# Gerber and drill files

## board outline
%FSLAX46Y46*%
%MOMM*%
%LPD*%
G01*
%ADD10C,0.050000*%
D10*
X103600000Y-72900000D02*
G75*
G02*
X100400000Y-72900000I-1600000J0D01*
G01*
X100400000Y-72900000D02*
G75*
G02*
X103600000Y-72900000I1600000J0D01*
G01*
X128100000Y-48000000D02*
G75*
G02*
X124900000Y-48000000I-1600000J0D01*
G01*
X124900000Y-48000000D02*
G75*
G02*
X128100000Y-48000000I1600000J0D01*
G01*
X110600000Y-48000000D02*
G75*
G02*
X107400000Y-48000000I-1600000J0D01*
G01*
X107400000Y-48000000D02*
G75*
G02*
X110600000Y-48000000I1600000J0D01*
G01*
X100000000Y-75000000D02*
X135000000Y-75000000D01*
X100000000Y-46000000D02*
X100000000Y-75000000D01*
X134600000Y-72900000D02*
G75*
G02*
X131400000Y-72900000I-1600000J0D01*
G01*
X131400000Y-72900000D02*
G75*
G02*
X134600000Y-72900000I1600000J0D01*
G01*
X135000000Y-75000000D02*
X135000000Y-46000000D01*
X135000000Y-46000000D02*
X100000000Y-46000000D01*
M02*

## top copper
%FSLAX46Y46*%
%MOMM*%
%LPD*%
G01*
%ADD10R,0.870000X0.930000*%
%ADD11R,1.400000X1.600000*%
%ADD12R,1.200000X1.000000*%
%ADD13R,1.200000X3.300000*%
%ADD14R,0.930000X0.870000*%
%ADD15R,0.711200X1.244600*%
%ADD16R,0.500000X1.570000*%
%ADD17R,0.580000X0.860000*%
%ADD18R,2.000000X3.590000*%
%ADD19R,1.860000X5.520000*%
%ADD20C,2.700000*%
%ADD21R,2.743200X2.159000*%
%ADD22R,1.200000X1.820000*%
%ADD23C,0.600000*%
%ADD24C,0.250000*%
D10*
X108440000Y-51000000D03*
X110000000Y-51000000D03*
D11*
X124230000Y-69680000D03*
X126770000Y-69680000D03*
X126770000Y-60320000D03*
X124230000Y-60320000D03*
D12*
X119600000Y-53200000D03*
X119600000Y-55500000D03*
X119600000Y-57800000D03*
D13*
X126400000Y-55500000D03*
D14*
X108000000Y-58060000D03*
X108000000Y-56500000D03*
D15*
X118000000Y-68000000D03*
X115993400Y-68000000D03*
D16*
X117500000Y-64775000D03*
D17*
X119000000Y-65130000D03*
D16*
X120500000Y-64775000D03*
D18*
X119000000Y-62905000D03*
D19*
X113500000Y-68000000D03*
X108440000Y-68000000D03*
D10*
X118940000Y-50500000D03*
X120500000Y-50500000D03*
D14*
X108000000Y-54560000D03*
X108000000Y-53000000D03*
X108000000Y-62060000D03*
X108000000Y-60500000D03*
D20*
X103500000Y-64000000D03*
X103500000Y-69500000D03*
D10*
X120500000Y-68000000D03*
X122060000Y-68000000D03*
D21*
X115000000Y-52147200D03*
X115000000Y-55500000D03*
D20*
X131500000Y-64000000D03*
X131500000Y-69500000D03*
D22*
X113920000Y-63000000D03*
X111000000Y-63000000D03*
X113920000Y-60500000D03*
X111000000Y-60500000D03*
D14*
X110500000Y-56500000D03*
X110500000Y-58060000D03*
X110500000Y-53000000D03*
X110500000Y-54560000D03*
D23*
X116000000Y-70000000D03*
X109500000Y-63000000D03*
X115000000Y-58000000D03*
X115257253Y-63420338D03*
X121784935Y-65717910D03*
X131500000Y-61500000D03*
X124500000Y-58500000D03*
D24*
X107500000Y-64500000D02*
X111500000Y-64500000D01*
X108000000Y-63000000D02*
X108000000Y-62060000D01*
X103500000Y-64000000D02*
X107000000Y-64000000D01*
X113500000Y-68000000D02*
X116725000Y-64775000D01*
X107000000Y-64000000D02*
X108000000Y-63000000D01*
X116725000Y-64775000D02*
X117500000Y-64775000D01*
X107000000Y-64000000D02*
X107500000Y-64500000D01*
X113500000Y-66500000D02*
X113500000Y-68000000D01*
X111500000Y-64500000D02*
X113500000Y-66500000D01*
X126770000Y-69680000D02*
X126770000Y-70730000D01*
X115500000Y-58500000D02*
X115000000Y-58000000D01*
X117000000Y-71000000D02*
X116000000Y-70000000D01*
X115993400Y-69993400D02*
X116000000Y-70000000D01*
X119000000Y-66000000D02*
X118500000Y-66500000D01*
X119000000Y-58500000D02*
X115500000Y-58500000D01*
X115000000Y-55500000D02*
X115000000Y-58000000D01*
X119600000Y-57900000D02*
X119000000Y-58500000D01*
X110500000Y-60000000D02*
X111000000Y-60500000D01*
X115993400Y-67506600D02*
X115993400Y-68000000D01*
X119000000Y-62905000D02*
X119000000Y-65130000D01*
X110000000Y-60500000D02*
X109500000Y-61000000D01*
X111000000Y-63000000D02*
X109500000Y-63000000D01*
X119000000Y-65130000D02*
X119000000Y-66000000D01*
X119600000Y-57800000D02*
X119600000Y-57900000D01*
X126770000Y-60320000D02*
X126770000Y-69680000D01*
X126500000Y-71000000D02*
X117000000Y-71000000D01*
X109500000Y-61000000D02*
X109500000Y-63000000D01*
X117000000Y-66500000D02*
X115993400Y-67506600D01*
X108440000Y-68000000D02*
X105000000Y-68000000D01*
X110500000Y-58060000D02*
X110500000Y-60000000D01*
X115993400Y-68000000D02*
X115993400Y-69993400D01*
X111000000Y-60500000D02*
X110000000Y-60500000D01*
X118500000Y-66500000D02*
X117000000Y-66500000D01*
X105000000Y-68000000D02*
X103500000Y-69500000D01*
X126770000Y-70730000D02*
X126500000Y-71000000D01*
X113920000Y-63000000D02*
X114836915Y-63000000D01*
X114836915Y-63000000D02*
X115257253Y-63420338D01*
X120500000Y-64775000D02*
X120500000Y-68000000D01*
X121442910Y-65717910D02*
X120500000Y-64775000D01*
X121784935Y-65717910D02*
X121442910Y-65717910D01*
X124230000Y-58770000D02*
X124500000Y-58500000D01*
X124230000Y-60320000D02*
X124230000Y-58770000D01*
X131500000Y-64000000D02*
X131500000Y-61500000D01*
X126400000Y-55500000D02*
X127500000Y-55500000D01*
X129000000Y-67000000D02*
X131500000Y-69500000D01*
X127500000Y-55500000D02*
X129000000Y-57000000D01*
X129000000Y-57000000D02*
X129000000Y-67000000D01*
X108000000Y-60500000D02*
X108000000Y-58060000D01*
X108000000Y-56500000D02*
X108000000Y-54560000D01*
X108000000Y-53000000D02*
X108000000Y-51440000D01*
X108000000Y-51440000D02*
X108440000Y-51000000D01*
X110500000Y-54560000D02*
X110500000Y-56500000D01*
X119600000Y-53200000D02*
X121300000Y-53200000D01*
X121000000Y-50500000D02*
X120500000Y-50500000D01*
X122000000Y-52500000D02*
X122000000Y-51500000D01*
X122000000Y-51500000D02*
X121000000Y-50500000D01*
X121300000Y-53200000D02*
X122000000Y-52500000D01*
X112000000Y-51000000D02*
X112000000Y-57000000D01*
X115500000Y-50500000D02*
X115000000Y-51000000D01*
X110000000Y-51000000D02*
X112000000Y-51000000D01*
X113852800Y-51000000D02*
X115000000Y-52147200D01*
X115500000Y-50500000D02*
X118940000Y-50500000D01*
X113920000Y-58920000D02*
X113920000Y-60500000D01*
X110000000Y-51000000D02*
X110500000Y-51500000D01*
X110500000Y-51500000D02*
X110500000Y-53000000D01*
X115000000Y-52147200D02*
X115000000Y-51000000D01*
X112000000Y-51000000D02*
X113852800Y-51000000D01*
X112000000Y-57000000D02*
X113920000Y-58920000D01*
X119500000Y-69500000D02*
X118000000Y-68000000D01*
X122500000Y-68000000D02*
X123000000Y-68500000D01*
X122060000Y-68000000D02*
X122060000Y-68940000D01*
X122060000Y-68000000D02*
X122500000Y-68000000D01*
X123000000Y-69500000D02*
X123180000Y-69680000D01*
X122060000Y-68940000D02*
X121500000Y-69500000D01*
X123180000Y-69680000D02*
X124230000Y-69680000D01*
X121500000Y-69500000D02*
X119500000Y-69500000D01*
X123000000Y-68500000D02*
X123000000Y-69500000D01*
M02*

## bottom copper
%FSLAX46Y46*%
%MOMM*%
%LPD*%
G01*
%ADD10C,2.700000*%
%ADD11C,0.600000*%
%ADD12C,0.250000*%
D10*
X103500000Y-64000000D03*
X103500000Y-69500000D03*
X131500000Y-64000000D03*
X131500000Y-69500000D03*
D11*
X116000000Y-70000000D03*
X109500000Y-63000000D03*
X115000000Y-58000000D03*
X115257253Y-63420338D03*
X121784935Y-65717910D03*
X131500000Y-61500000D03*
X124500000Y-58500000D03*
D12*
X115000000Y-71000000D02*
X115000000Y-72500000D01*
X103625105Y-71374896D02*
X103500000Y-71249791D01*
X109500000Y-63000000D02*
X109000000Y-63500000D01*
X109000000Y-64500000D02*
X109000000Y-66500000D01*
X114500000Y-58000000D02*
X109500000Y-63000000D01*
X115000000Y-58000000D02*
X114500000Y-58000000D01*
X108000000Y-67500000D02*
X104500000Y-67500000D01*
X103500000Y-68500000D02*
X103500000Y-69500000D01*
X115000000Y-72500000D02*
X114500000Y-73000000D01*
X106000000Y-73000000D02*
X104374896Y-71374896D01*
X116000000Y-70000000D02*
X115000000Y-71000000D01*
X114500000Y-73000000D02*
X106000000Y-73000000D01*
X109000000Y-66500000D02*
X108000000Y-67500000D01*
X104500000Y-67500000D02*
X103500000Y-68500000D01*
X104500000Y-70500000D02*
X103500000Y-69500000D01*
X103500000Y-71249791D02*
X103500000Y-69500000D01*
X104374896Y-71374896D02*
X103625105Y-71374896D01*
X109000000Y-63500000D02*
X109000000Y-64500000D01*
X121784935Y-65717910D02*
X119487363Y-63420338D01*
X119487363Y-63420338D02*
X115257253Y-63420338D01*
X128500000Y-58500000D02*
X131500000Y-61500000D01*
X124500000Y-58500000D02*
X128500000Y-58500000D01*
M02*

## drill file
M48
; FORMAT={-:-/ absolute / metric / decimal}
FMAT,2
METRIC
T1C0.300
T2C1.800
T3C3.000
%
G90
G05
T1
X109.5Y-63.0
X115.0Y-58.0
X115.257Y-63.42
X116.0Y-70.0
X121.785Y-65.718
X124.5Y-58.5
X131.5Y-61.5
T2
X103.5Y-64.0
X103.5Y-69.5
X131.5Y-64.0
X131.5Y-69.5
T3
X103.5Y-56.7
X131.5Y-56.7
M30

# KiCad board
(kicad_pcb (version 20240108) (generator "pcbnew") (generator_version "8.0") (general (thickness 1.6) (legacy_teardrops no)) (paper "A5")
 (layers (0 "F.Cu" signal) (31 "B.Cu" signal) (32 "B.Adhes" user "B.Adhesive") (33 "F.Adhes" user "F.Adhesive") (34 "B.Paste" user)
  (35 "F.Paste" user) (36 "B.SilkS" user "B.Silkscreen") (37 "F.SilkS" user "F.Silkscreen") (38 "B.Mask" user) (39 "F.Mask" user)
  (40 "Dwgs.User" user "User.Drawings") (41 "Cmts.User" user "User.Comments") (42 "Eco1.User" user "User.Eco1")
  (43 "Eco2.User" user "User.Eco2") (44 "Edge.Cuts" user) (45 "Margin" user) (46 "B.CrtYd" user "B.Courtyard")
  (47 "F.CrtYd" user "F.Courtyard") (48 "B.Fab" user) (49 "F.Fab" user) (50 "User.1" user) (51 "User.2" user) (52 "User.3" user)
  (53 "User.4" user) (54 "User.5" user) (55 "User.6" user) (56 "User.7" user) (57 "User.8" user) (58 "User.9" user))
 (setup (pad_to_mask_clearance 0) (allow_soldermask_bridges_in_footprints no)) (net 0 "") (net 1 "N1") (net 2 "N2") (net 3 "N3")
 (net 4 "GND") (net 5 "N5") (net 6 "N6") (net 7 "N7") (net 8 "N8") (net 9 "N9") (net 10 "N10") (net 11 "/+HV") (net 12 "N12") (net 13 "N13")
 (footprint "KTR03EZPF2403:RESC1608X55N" (layer "F.Cu") (at 109.22 51)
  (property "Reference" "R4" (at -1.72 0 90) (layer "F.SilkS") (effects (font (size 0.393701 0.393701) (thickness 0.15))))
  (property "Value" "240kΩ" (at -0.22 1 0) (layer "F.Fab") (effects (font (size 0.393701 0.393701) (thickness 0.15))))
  (pad "1" smd rect (at -0.78 0) (size 0.87 0.93) (layers "F.Cu" "F.Paste" "F.Mask") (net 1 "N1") (solder_mask_margin 0.102))
  (pad "2" smd rect (at 0.78 0) (size 0.87 0.93) (layers "F.Cu" "F.Paste" "F.Mask") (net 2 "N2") (solder_mask_margin 0.102)))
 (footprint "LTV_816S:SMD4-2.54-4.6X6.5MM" (layer "F.Cu") (at 125.5 65)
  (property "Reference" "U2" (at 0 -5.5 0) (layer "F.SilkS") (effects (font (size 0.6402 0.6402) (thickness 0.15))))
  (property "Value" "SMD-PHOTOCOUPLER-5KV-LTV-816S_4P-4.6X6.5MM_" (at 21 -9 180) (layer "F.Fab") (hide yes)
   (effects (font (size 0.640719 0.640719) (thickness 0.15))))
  (pad "1" smd rect (at -1.27 4.68) (size 1.4 1.6) (layers "F.Cu" "F.Paste" "F.Mask") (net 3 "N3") (solder_mask_margin 0.102))
  (pad "2" smd rect (at 1.27 4.68) (size 1.4 1.6) (layers "F.Cu" "F.Paste" "F.Mask") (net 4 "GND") (solder_mask_margin 0.102))
  (pad "3" smd rect (at 1.27 -4.68) (size 1.4 1.6) (layers "F.Cu" "F.Paste" "F.Mask") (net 4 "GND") (solder_mask_margin 0.102))
  (pad "4" smd rect (at -1.27 -4.68) (size 1.4 1.6) (layers "F.Cu" "F.Paste" "F.Mask") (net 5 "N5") (solder_mask_margin 0.102)))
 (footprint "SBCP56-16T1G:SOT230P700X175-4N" (layer "F.Cu") (at 123 55.5)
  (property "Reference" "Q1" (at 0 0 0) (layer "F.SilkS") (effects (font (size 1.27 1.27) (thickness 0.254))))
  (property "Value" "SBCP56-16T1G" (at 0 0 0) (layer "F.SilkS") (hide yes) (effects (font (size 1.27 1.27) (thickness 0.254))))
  (pad "1" smd rect (at -3.4 -2.3 90) (size 1 1.2) (layers "F.Cu" "F.Paste" "F.Mask") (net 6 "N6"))
  (pad "2" smd rect (at -3.4 0 90) (size 1 1.2) (layers "F.Cu" "F.Paste" "F.Mask") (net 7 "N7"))
  (pad "3" smd rect (at -3.4 2.3 90) (size 1 1.2) (layers "F.Cu" "F.Paste" "F.Mask") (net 4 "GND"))
  (pad "4" smd rect (at 3.4 0) (size 1.2 3.3) (layers "F.Cu" "F.Paste" "F.Mask") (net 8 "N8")))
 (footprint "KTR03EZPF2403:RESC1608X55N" (layer "F.Cu") (at 108 57.28 90)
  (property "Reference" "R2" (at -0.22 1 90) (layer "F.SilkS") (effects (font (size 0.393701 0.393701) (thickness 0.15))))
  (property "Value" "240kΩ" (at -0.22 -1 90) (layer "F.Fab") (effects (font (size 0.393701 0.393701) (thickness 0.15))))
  (pad "1" smd rect (at -0.78 0 90) (size 0.87 0.93) (layers "F.Cu" "F.Paste" "F.Mask") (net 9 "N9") (solder_mask_margin 0.102))
  (pad "2" smd rect (at 0.78 0 90) (size 0.87 0.93) (layers "F.Cu" "F.Paste" "F.Mask") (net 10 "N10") (solder_mask_margin 0.102)))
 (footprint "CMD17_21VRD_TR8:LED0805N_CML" (layer "F.Cu") (at 116.9967 68 180)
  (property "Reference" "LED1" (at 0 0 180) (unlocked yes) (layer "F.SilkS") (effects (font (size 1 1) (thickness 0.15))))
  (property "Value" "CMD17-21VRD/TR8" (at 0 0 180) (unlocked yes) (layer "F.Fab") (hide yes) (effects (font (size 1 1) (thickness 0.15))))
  (pad "1" smd rect (at -1.0033 0 180) (size 0.7112 1.2446) (layers "F.Cu" "F.Paste" "F.Mask") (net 3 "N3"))
  (pad "2" smd rect (at 1.0033 0 180) (size 0.7112 1.2446) (layers "F.Cu" "F.Paste" "F.Mask") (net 4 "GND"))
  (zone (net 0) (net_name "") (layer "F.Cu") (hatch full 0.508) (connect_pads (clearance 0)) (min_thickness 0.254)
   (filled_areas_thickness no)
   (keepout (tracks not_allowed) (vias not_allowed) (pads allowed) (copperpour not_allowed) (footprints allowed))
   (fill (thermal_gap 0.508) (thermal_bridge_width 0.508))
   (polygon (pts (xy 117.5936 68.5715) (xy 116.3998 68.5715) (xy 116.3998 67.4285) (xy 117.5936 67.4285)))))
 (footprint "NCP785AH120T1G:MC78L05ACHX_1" (layer "F.Cu") (at 119 64.5)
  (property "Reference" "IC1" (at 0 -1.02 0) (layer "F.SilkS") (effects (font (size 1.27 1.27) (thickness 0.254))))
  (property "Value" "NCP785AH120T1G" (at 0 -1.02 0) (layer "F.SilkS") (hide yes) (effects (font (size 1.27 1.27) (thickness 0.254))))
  (pad "1" smd rect (at -1.5 0.275) (size 0.5 1.57) (layers "F.Cu" "F.Paste" "F.Mask") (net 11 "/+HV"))
  (pad "2" smd rect (at 0 0.63) (size 0.58 0.86) (layers "F.Cu" "F.Paste" "F.Mask") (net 4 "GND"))
  (pad "3" smd rect (at 1.5 0.275) (size 0.5 1.57) (layers "F.Cu" "F.Paste" "F.Mask") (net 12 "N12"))
  (pad "4" smd rect (at 0 -1.595) (size 2 3.59) (layers "F.Cu" "F.Paste" "F.Mask") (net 4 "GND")))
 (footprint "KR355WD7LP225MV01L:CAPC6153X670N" (layer "F.Cu") (at 110.97 68 180)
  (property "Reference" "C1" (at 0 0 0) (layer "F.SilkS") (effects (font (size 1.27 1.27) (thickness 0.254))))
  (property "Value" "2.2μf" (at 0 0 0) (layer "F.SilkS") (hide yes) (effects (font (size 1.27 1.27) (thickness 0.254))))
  (pad "1" smd rect (at -2.53 0 180) (size 1.86 5.52) (layers "F.Cu" "F.Paste" "F.Mask") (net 11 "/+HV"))
  (pad "2" smd rect (at 2.53 0 180) (size 1.86 5.52) (layers "F.Cu" "F.Paste" "F.Mask") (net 4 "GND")))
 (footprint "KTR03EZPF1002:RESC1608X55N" (layer "F.Cu") (at 119.72 50.5)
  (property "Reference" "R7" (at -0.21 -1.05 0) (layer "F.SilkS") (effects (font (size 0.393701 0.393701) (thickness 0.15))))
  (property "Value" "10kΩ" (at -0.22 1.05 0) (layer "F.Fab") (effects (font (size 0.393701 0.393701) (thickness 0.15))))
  (pad "1" smd rect (at -0.78 0) (size 0.87 0.93) (layers "F.Cu" "F.Paste" "F.Mask") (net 2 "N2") (solder_mask_margin 0.102))
  (pad "2" smd rect (at 0.78 0) (size 0.87 0.93) (layers "F.Cu" "F.Paste" "F.Mask") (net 6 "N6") (solder_mask_margin 0.102)))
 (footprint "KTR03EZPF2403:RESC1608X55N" (layer "F.Cu") (at 108 53.78 90)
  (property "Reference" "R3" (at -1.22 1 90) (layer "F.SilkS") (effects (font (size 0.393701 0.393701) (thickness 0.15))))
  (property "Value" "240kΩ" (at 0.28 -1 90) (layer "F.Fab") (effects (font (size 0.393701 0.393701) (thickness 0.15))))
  (pad "1" smd rect (at -0.78 0 90) (size 0.87 0.93) (layers "F.Cu" "F.Paste" "F.Mask") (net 10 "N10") (solder_mask_margin 0.102))
  (pad "2" smd rect (at 0.78 0 90) (size 0.87 0.93) (layers "F.Cu" "F.Paste" "F.Mask") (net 1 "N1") (solder_mask_margin 0.102)))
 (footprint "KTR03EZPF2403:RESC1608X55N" (layer "F.Cu") (at 108 61.28 90)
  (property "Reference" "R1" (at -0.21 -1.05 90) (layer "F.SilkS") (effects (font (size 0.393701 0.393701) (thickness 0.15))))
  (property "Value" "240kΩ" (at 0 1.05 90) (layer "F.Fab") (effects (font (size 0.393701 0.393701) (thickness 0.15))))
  (pad "1" smd rect (at -0.78 0 90) (size 0.87 0.93) (layers "F.Cu" "F.Paste" "F.Mask") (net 11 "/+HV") (solder_mask_margin 0.102))
  (pad "2" smd rect (at 0.78 0 90) (size 0.87 0.93) (layers "F.Cu" "F.Paste" "F.Mask") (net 9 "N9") (solder_mask_margin 0.102)))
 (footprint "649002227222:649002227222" (layer "F.Cu") (at 103.5 56.5 180)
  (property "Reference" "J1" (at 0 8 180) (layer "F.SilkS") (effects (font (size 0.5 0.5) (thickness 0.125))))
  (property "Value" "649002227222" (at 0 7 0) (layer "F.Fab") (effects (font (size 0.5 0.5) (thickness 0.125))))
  (pad "" np_thru_hole circle (at 0 -0.2 180) (size 3 3) (drill 3) (layers "*.Cu" "*.Mask"))
  (pad "1" thru_hole circle (at 0 -7.5 180) (size 2.7 2.7) (drill 1.8) (layers "*.Cu" "*.Mask") (remove_unused_layers no) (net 11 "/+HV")
   (solder_mask_margin 0.102))
  (pad "2" thru_hole circle (at 0 -13 180) (size 2.7 2.7) (drill 1.8) (layers "*.Cu" "*.Mask") (remove_unused_layers no) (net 4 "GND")
   (solder_mask_margin 0.102)))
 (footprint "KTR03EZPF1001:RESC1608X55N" (layer "F.Cu") (at 121.28 68)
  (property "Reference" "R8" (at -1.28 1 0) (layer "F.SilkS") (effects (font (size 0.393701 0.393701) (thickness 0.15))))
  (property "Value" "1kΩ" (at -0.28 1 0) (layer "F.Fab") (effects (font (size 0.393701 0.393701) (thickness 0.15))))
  (pad "1" smd rect (at -0.78 0) (size 0.87 0.93) (layers "F.Cu" "F.Paste" "F.Mask") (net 12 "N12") (solder_mask_margin 0.102))
  (pad "2" smd rect (at 0.78 0) (size 0.87 0.93) (layers "F.Cu" "F.Paste" "F.Mask") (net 3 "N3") (solder_mask_margin 0.102)))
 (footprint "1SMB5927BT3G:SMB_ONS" (layer "F.Cu") (at 115 53.8236 -90)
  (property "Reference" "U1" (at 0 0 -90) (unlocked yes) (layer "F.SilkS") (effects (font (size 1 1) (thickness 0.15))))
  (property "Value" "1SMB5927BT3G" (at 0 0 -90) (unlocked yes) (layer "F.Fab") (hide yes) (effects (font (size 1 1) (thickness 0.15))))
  (pad "1" smd rect (at -1.6764 0 270) (size 2.159 2.7432) (layers "F.Cu" "F.Paste" "F.Mask") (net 2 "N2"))
  (pad "2" smd rect (at 1.6764 0 270) (size 2.159 2.7432) (layers "F.Cu" "F.Paste" "F.Mask") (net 4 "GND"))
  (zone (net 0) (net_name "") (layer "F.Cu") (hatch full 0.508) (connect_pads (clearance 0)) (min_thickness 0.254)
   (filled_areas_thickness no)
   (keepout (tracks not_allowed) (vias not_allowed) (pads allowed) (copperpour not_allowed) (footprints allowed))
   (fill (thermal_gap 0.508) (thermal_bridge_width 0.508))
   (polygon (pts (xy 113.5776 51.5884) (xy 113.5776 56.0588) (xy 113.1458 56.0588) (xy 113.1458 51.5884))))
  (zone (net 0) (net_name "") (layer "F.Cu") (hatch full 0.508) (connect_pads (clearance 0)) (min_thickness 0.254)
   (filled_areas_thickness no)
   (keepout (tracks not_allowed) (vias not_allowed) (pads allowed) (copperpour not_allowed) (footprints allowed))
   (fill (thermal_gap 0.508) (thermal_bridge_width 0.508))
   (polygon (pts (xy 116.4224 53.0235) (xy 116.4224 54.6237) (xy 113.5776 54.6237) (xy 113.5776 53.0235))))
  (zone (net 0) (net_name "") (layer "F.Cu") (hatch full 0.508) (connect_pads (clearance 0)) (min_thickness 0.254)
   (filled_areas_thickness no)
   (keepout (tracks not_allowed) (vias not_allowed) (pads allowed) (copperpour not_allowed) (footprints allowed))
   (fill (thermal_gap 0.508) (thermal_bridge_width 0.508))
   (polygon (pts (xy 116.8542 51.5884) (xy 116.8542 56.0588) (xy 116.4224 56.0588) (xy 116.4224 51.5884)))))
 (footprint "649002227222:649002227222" (layer "F.Cu") (at 131.5 56.5 180)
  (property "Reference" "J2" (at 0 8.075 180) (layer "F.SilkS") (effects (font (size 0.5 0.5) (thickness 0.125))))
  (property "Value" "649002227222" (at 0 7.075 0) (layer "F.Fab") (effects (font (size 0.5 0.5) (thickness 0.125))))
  (pad "" np_thru_hole circle (at 0 -0.2 180) (size 3 3) (drill 3) (layers "*.Cu" "*.Mask"))
  (pad "1" thru_hole circle (at 0 -7.5 180) (size 2.7 2.7) (drill 1.8) (layers "*.Cu" "*.Mask") (remove_unused_layers no) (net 5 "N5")
   (solder_mask_margin 0.102))
  (pad "2" thru_hole circle (at 0 -13 180) (size 2.7 2.7) (drill 1.8) (layers "*.Cu" "*.Mask") (remove_unused_layers no) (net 8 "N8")
   (solder_mask_margin 0.102)))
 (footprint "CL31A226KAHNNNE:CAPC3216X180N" (layer "F.Cu") (at 112.46 63 180)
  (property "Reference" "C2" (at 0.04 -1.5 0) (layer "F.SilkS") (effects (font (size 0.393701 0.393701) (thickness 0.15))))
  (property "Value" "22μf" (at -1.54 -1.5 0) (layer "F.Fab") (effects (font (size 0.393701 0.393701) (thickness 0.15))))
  (pad "1" smd rect (at -1.46 0 180) (size 1.2 1.82) (layers "F.Cu" "F.Paste" "F.Mask") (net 12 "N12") (solder_mask_margin 0.102))
  (pad "2" smd rect (at 1.46 0 180) (size 1.2 1.82) (layers "F.Cu" "F.Paste" "F.Mask") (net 4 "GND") (solder_mask_margin 0.102)))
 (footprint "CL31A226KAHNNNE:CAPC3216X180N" (layer "F.Cu") (at 112.46 60.5 180)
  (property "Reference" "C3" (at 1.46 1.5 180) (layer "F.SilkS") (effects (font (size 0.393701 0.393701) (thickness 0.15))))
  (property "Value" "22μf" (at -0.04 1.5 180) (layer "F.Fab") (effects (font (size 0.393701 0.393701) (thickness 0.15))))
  (pad "1" smd rect (at -1.46 0 180) (size 1.2 1.82) (layers "F.Cu" "F.Paste" "F.Mask") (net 2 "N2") (solder_mask_margin 0.102))
  (pad "2" smd rect (at 1.46 0 180) (size 1.2 1.82) (layers "F.Cu" "F.Paste" "F.Mask") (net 4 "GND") (solder_mask_margin 0.102)))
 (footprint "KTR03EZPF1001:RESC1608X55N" (layer "F.Cu") (at 110.5 57.28 -90)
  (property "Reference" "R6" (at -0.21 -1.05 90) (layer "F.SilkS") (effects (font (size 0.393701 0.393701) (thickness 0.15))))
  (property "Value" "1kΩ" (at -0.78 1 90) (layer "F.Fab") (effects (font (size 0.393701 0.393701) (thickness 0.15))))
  (pad "1" smd rect (at -0.78 0 270) (size 0.87 0.93) (layers "F.Cu" "F.Paste" "F.Mask") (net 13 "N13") (solder_mask_margin 0.102))
  (pad "2" smd rect (at 0.78 0 270) (size 0.87 0.93) (layers "F.Cu" "F.Paste" "F.Mask") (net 4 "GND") (solder_mask_margin 0.102)))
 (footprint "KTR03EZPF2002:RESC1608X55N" (layer "F.Cu") (at 110.5 53.78 -90)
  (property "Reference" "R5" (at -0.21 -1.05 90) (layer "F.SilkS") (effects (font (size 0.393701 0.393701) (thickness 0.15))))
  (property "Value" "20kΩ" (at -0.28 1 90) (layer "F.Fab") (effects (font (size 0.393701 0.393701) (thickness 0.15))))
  (pad "1" smd rect (at -0.78 0 270) (size 0.87 0.93) (layers "F.Cu" "F.Paste" "F.Mask") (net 2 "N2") (solder_mask_margin 0.102))
  (pad "2" smd rect (at 0.78 0 270) (size 0.87 0.93) (layers "F.Cu" "F.Paste" "F.Mask") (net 13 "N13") (solder_mask_margin 0.102)))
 (gr_circle (center 102 72.9) (end 102 74.5) (stroke (width 0.05) (type default)) (fill none) (layer "Edge.Cuts"))
 (gr_circle (center 126.5 48) (end 128.1 48) (stroke (width 0.05) (type default)) (fill none) (layer "Edge.Cuts"))
 (gr_circle (center 109 48) (end 110.6 48) (stroke (width 0.05) (type default)) (fill none) (layer "Edge.Cuts"))
 (gr_line (start 100 75) (end 135 75) (stroke (width 0.05) (type default)) (layer "Edge.Cuts"))
 (gr_line (start 100 46) (end 100 75) (stroke (width 0.05) (type default)) (layer "Edge.Cuts"))
 (gr_circle (center 133 72.9) (end 134.6 72.9) (stroke (width 0.05) (type default)) (fill none) (layer "Edge.Cuts"))
 (gr_line (start 135 75) (end 135 46) (stroke (width 0.05) (type default)) (layer "Edge.Cuts"))
 (gr_line (start 135 46) (end 100 46) (stroke (width 0.05) (type default)) (layer "Edge.Cuts"))
 (segment (start 107.5 64.5) (end 111.5 64.5) (width 0.25) (layer "F.Cu") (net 11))
 (segment (start 108 63) (end 108 62.06) (width 0.25) (layer "F.Cu") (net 11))
 (segment (start 103.5 64) (end 107 64) (width 0.25) (layer "F.Cu") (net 11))
 (segment (start 113.5 68) (end 116.725 64.775) (width 0.25) (layer "F.Cu") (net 11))
 (segment (start 107 64) (end 108 63) (width 0.25) (layer "F.Cu") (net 11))
 (segment (start 116.725 64.775) (end 117.5 64.775) (width 0.25) (layer "F.Cu") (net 11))
 (segment (start 107 64) (end 107.5 64.5) (width 0.25) (layer "F.Cu") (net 11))
 (segment (start 113.5 66.5) (end 113.5 68) (width 0.25) (layer "F.Cu") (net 11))
 (segment (start 111.5 64.5) (end 113.5 66.5) (width 0.25) (layer "F.Cu") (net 11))
 (segment (start 126.77 69.68) (end 126.77 70.73) (width 0.25) (layer "F.Cu") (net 4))
 (segment (start 115.5 58.5) (end 115 58) (width 0.25) (layer "F.Cu") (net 4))
 (segment (start 117 71) (end 116 70) (width 0.25) (layer "F.Cu") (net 4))
 (segment (start 115.9934 69.9934) (end 116 70) (width 0.25) (layer "F.Cu") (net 4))
 (segment (start 119 66) (end 118.5 66.5) (width 0.25) (layer "F.Cu") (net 4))
 (segment (start 119 58.5) (end 115.5 58.5) (width 0.25) (layer "F.Cu") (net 4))
 (segment (start 115 55.5) (end 115 58) (width 0.25) (layer "F.Cu") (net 4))
 (segment (start 119.6 57.9) (end 119 58.5) (width 0.25) (layer "F.Cu") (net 4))
 (segment (start 110.5 60) (end 111 60.5) (width 0.25) (layer "F.Cu") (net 4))
 (segment (start 115.9934 67.5066) (end 115.9934 68) (width 0.25) (layer "F.Cu") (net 4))
 (segment (start 119 62.905) (end 119 65.13) (width 0.25) (layer "F.Cu") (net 4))
 (segment (start 110 60.5) (end 109.5 61) (width 0.25) (layer "F.Cu") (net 4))
 (segment (start 111 63) (end 109.5 63) (width 0.25) (layer "F.Cu") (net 4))
 (segment (start 119 65.13) (end 119 66) (width 0.25) (layer "F.Cu") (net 4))
 (segment (start 119.6 57.8) (end 119.6 57.9) (width 0.25) (layer "F.Cu") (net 4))
 (segment (start 126.77 60.32) (end 126.77 69.68) (width 0.25) (layer "F.Cu") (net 4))
 (segment (start 126.5 71) (end 117 71) (width 0.25) (layer "F.Cu") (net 4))
 (segment (start 109.5 61) (end 109.5 63) (width 0.25) (layer "F.Cu") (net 4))
 (segment (start 117 66.5) (end 115.9934 67.5066) (width 0.25) (layer "F.Cu") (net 4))
 (segment (start 108.44 68) (end 105 68) (width 0.25) (layer "F.Cu") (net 4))
 (segment (start 110.5 58.06) (end 110.5 60) (width 0.25) (layer "F.Cu") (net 4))
 (segment (start 115.9934 68) (end 115.9934 69.9934) (width 0.25) (layer "F.Cu") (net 4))
 (segment (start 111 60.5) (end 110 60.5) (width 0.25) (layer "F.Cu") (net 4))
 (segment (start 118.5 66.5) (end 117 66.5) (width 0.25) (layer "F.Cu") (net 4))
 (segment (start 105 68) (end 103.5 69.5) (width 0.25) (layer "F.Cu") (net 4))
 (segment (start 126.77 70.73) (end 126.5 71) (width 0.25) (layer "F.Cu") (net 4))
 (via (at 116 70) (size 0.6) (drill 0.3) (layers "F.Cu" "B.Cu") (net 4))
 (via (at 109.5 63) (size 0.6) (drill 0.3) (layers "F.Cu" "B.Cu") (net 4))
 (via (at 115 58) (size 0.6) (drill 0.3) (layers "F.Cu" "B.Cu") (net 4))
 (segment (start 115 71) (end 115 72.5) (width 0.25) (layer "B.Cu") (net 4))
 (segment (start 103.625105 71.374896) (end 103.5 71.249791) (width 0.25) (layer "B.Cu") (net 4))
 (segment (start 109.5 63) (end 109 63.5) (width 0.25) (layer "B.Cu") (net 4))
 (segment (start 109 64.5) (end 109 66.5) (width 0.25) (layer "B.Cu") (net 4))
 (segment (start 114.5 58) (end 109.5 63) (width 0.25) (layer "B.Cu") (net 4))
 (segment (start 115 58) (end 114.5 58) (width 0.25) (layer "B.Cu") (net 4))
 (segment (start 108 67.5) (end 104.5 67.5) (width 0.25) (layer "B.Cu") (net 4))
 (segment (start 103.5 68.5) (end 103.5 69.5) (width 0.25) (layer "B.Cu") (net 4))
 (segment (start 115 72.5) (end 114.5 73) (width 0.25) (layer "B.Cu") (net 4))
 (segment (start 106 73) (end 104.374896 71.374896) (width 0.25) (layer "B.Cu") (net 4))
 (segment (start 116 70) (end 115 71) (width 0.25) (layer "B.Cu") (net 4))
 (segment (start 114.5 73) (end 106 73) (width 0.25) (layer "B.Cu") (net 4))
 (segment (start 109 66.5) (end 108 67.5) (width 0.25) (layer "B.Cu") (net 4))
 (segment (start 104.5 67.5) (end 103.5 68.5) (width 0.25) (layer "B.Cu") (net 4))
 (segment (start 104.5 70.5) (end 103.5 69.5) (width 0.25) (layer "B.Cu") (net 4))
 (segment (start 103.5 71.249791) (end 103.5 69.5) (width 0.25) (layer "B.Cu") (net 4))
 (segment (start 104.374896 71.374896) (end 103.625105 71.374896) (width 0.25) (layer "B.Cu") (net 4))
 (segment (start 109 63.5) (end 109 64.5) (width 0.25) (layer "B.Cu") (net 4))
 (segment (start 113.92 63) (end 114.836915 63) (width 0.25) (layer "F.Cu") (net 12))
 (segment (start 114.836915 63) (end 115.257253 63.420338) (width 0.25) (layer "F.Cu") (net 12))
 (segment (start 120.5 64.775) (end 120.5 68) (width 0.25) (layer "F.Cu") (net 12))
 (segment (start 121.44291 65.71791) (end 120.5 64.775) (width 0.25) (layer "F.Cu") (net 12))
 (segment (start 121.784935 65.71791) (end 121.44291 65.71791) (width 0.25) (layer "F.Cu") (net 12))
 (via (at 115.257253 63.420338) (size 0.6) (drill 0.3) (layers "F.Cu" "B.Cu") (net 12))
 (via (at 121.784935 65.71791) (size 0.6) (drill 0.3) (layers "F.Cu" "B.Cu") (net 12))
 (segment (start 121.784935 65.71791) (end 119.487363 63.420338) (width 0.25) (layer "B.Cu") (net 12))
 (segment (start 119.487363 63.420338) (end 115.257253 63.420338) (width 0.25) (layer "B.Cu") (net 12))
 (segment (start 124.23 58.77) (end 124.5 58.5) (width 0.25) (layer "F.Cu") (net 5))
 (segment (start 124.23 60.32) (end 124.23 58.77) (width 0.25) (layer "F.Cu") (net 5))
 (segment (start 131.5 64) (end 131.5 61.5) (width 0.25) (layer "F.Cu") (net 5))
 (via (at 131.5 61.5) (size 0.6) (drill 0.3) (layers "F.Cu" "B.Cu") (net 5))
 (via (at 124.5 58.5) (size 0.6) (drill 0.3) (layers "F.Cu" "B.Cu") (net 5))
 (segment (start 128.5 58.5) (end 131.5 61.5) (width 0.25) (layer "B.Cu") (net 5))
 (segment (start 124.5 58.5) (end 128.5 58.5) (width 0.25) (layer "B.Cu") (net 5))
 (segment (start 126.4 55.5) (end 127.5 55.5) (width 0.25) (layer "F.Cu") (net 8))
 (segment (start 129 67) (end 131.5 69.5) (width 0.25) (layer "F.Cu") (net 8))
 (segment (start 127.5 55.5) (end 129 57) (width 0.25) (layer "F.Cu") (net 8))
 (segment (start 129 57) (end 129 67) (width 0.25) (layer "F.Cu") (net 8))
 (segment (start 108 60.5) (end 108 58.06) (width 0.25) (layer "F.Cu") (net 9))
 (segment (start 108 56.5) (end 108 54.56) (width 0.25) (layer "F.Cu") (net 10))
 (segment (start 108 53) (end 108 51.44) (width 0.25) (layer "F.Cu") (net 1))
 (segment (start 108 51.44) (end 108.44 51) (width 0.25) (layer "F.Cu") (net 1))
 (segment (start 110.5 54.56) (end 110.5 56.5) (width 0.25) (layer "F.Cu") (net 13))
 (segment (start 119.6 53.2) (end 121.3 53.2) (width 0.25) (layer "F.Cu") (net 6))
 (segment (start 121 50.5) (end 120.5 50.5) (width 0.25) (layer "F.Cu") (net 6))
 (segment (start 122 52.5) (end 122 51.5) (width 0.25) (layer "F.Cu") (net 6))
 (segment (start 122 51.5) (end 121 50.5) (width 0.25) (layer "F.Cu") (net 6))
 (segment (start 121.3 53.2) (end 122 52.5) (width 0.25) (layer "F.Cu") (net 6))
 (segment (start 112 51) (end 112 57) (width 0.25) (layer "F.Cu") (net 2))
 (segment (start 115.5 50.5) (end 115 51) (width 0.25) (layer "F.Cu") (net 2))
 (segment (start 110 51) (end 112 51) (width 0.25) (layer "F.Cu") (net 2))
 (segment (start 113.8528 51) (end 115 52.1472) (width 0.25) (layer "F.Cu") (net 2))
 (segment (start 115.5 50.5) (end 118.94 50.5) (width 0.25) (layer "F.Cu") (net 2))
 (segment (start 113.92 58.92) (end 113.92 60.5) (width 0.25) (layer "F.Cu") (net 2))
 (segment (start 110 51) (end 110.5 51.5) (width 0.25) (layer "F.Cu") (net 2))
 (segment (start 110.5 51.5) (end 110.5 53) (width 0.25) (layer "F.Cu") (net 2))
 (segment (start 115 52.1472) (end 115 51) (width 0.25) (layer "F.Cu") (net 2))
 (segment (start 112 51) (end 113.8528 51) (width 0.25) (layer "F.Cu") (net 2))
 (segment (start 112 57) (end 113.92 58.92) (width 0.25) (layer "F.Cu") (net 2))
 (segment (start 119.5 69.5) (end 118 68) (width 0.25) (layer "F.Cu") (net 3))
 (segment (start 122.5 68) (end 123 68.5) (width 0.25) (layer "F.Cu") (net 3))
 (segment (start 122.06 68) (end 122.06 68.94) (width 0.25) (layer "F.Cu") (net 3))
 (segment (start 122.06 68) (end 122.5 68) (width 0.25) (layer "F.Cu") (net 3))
 (segment (start 123 69.5) (end 123.18 69.68) (width 0.25) (layer "F.Cu") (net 3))
 (segment (start 122.06 68.94) (end 121.5 69.5) (width 0.25) (layer "F.Cu") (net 3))
 (segment (start 123.18 69.68) (end 124.23 69.68) (width 0.25) (layer "F.Cu") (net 3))
 (segment (start 121.5 69.5) (end 119.5 69.5) (width 0.25) (layer "F.Cu") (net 3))
 (segment (start 123 68.5) (end 123 69.5) (width 0.25) (layer "F.Cu") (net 3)))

